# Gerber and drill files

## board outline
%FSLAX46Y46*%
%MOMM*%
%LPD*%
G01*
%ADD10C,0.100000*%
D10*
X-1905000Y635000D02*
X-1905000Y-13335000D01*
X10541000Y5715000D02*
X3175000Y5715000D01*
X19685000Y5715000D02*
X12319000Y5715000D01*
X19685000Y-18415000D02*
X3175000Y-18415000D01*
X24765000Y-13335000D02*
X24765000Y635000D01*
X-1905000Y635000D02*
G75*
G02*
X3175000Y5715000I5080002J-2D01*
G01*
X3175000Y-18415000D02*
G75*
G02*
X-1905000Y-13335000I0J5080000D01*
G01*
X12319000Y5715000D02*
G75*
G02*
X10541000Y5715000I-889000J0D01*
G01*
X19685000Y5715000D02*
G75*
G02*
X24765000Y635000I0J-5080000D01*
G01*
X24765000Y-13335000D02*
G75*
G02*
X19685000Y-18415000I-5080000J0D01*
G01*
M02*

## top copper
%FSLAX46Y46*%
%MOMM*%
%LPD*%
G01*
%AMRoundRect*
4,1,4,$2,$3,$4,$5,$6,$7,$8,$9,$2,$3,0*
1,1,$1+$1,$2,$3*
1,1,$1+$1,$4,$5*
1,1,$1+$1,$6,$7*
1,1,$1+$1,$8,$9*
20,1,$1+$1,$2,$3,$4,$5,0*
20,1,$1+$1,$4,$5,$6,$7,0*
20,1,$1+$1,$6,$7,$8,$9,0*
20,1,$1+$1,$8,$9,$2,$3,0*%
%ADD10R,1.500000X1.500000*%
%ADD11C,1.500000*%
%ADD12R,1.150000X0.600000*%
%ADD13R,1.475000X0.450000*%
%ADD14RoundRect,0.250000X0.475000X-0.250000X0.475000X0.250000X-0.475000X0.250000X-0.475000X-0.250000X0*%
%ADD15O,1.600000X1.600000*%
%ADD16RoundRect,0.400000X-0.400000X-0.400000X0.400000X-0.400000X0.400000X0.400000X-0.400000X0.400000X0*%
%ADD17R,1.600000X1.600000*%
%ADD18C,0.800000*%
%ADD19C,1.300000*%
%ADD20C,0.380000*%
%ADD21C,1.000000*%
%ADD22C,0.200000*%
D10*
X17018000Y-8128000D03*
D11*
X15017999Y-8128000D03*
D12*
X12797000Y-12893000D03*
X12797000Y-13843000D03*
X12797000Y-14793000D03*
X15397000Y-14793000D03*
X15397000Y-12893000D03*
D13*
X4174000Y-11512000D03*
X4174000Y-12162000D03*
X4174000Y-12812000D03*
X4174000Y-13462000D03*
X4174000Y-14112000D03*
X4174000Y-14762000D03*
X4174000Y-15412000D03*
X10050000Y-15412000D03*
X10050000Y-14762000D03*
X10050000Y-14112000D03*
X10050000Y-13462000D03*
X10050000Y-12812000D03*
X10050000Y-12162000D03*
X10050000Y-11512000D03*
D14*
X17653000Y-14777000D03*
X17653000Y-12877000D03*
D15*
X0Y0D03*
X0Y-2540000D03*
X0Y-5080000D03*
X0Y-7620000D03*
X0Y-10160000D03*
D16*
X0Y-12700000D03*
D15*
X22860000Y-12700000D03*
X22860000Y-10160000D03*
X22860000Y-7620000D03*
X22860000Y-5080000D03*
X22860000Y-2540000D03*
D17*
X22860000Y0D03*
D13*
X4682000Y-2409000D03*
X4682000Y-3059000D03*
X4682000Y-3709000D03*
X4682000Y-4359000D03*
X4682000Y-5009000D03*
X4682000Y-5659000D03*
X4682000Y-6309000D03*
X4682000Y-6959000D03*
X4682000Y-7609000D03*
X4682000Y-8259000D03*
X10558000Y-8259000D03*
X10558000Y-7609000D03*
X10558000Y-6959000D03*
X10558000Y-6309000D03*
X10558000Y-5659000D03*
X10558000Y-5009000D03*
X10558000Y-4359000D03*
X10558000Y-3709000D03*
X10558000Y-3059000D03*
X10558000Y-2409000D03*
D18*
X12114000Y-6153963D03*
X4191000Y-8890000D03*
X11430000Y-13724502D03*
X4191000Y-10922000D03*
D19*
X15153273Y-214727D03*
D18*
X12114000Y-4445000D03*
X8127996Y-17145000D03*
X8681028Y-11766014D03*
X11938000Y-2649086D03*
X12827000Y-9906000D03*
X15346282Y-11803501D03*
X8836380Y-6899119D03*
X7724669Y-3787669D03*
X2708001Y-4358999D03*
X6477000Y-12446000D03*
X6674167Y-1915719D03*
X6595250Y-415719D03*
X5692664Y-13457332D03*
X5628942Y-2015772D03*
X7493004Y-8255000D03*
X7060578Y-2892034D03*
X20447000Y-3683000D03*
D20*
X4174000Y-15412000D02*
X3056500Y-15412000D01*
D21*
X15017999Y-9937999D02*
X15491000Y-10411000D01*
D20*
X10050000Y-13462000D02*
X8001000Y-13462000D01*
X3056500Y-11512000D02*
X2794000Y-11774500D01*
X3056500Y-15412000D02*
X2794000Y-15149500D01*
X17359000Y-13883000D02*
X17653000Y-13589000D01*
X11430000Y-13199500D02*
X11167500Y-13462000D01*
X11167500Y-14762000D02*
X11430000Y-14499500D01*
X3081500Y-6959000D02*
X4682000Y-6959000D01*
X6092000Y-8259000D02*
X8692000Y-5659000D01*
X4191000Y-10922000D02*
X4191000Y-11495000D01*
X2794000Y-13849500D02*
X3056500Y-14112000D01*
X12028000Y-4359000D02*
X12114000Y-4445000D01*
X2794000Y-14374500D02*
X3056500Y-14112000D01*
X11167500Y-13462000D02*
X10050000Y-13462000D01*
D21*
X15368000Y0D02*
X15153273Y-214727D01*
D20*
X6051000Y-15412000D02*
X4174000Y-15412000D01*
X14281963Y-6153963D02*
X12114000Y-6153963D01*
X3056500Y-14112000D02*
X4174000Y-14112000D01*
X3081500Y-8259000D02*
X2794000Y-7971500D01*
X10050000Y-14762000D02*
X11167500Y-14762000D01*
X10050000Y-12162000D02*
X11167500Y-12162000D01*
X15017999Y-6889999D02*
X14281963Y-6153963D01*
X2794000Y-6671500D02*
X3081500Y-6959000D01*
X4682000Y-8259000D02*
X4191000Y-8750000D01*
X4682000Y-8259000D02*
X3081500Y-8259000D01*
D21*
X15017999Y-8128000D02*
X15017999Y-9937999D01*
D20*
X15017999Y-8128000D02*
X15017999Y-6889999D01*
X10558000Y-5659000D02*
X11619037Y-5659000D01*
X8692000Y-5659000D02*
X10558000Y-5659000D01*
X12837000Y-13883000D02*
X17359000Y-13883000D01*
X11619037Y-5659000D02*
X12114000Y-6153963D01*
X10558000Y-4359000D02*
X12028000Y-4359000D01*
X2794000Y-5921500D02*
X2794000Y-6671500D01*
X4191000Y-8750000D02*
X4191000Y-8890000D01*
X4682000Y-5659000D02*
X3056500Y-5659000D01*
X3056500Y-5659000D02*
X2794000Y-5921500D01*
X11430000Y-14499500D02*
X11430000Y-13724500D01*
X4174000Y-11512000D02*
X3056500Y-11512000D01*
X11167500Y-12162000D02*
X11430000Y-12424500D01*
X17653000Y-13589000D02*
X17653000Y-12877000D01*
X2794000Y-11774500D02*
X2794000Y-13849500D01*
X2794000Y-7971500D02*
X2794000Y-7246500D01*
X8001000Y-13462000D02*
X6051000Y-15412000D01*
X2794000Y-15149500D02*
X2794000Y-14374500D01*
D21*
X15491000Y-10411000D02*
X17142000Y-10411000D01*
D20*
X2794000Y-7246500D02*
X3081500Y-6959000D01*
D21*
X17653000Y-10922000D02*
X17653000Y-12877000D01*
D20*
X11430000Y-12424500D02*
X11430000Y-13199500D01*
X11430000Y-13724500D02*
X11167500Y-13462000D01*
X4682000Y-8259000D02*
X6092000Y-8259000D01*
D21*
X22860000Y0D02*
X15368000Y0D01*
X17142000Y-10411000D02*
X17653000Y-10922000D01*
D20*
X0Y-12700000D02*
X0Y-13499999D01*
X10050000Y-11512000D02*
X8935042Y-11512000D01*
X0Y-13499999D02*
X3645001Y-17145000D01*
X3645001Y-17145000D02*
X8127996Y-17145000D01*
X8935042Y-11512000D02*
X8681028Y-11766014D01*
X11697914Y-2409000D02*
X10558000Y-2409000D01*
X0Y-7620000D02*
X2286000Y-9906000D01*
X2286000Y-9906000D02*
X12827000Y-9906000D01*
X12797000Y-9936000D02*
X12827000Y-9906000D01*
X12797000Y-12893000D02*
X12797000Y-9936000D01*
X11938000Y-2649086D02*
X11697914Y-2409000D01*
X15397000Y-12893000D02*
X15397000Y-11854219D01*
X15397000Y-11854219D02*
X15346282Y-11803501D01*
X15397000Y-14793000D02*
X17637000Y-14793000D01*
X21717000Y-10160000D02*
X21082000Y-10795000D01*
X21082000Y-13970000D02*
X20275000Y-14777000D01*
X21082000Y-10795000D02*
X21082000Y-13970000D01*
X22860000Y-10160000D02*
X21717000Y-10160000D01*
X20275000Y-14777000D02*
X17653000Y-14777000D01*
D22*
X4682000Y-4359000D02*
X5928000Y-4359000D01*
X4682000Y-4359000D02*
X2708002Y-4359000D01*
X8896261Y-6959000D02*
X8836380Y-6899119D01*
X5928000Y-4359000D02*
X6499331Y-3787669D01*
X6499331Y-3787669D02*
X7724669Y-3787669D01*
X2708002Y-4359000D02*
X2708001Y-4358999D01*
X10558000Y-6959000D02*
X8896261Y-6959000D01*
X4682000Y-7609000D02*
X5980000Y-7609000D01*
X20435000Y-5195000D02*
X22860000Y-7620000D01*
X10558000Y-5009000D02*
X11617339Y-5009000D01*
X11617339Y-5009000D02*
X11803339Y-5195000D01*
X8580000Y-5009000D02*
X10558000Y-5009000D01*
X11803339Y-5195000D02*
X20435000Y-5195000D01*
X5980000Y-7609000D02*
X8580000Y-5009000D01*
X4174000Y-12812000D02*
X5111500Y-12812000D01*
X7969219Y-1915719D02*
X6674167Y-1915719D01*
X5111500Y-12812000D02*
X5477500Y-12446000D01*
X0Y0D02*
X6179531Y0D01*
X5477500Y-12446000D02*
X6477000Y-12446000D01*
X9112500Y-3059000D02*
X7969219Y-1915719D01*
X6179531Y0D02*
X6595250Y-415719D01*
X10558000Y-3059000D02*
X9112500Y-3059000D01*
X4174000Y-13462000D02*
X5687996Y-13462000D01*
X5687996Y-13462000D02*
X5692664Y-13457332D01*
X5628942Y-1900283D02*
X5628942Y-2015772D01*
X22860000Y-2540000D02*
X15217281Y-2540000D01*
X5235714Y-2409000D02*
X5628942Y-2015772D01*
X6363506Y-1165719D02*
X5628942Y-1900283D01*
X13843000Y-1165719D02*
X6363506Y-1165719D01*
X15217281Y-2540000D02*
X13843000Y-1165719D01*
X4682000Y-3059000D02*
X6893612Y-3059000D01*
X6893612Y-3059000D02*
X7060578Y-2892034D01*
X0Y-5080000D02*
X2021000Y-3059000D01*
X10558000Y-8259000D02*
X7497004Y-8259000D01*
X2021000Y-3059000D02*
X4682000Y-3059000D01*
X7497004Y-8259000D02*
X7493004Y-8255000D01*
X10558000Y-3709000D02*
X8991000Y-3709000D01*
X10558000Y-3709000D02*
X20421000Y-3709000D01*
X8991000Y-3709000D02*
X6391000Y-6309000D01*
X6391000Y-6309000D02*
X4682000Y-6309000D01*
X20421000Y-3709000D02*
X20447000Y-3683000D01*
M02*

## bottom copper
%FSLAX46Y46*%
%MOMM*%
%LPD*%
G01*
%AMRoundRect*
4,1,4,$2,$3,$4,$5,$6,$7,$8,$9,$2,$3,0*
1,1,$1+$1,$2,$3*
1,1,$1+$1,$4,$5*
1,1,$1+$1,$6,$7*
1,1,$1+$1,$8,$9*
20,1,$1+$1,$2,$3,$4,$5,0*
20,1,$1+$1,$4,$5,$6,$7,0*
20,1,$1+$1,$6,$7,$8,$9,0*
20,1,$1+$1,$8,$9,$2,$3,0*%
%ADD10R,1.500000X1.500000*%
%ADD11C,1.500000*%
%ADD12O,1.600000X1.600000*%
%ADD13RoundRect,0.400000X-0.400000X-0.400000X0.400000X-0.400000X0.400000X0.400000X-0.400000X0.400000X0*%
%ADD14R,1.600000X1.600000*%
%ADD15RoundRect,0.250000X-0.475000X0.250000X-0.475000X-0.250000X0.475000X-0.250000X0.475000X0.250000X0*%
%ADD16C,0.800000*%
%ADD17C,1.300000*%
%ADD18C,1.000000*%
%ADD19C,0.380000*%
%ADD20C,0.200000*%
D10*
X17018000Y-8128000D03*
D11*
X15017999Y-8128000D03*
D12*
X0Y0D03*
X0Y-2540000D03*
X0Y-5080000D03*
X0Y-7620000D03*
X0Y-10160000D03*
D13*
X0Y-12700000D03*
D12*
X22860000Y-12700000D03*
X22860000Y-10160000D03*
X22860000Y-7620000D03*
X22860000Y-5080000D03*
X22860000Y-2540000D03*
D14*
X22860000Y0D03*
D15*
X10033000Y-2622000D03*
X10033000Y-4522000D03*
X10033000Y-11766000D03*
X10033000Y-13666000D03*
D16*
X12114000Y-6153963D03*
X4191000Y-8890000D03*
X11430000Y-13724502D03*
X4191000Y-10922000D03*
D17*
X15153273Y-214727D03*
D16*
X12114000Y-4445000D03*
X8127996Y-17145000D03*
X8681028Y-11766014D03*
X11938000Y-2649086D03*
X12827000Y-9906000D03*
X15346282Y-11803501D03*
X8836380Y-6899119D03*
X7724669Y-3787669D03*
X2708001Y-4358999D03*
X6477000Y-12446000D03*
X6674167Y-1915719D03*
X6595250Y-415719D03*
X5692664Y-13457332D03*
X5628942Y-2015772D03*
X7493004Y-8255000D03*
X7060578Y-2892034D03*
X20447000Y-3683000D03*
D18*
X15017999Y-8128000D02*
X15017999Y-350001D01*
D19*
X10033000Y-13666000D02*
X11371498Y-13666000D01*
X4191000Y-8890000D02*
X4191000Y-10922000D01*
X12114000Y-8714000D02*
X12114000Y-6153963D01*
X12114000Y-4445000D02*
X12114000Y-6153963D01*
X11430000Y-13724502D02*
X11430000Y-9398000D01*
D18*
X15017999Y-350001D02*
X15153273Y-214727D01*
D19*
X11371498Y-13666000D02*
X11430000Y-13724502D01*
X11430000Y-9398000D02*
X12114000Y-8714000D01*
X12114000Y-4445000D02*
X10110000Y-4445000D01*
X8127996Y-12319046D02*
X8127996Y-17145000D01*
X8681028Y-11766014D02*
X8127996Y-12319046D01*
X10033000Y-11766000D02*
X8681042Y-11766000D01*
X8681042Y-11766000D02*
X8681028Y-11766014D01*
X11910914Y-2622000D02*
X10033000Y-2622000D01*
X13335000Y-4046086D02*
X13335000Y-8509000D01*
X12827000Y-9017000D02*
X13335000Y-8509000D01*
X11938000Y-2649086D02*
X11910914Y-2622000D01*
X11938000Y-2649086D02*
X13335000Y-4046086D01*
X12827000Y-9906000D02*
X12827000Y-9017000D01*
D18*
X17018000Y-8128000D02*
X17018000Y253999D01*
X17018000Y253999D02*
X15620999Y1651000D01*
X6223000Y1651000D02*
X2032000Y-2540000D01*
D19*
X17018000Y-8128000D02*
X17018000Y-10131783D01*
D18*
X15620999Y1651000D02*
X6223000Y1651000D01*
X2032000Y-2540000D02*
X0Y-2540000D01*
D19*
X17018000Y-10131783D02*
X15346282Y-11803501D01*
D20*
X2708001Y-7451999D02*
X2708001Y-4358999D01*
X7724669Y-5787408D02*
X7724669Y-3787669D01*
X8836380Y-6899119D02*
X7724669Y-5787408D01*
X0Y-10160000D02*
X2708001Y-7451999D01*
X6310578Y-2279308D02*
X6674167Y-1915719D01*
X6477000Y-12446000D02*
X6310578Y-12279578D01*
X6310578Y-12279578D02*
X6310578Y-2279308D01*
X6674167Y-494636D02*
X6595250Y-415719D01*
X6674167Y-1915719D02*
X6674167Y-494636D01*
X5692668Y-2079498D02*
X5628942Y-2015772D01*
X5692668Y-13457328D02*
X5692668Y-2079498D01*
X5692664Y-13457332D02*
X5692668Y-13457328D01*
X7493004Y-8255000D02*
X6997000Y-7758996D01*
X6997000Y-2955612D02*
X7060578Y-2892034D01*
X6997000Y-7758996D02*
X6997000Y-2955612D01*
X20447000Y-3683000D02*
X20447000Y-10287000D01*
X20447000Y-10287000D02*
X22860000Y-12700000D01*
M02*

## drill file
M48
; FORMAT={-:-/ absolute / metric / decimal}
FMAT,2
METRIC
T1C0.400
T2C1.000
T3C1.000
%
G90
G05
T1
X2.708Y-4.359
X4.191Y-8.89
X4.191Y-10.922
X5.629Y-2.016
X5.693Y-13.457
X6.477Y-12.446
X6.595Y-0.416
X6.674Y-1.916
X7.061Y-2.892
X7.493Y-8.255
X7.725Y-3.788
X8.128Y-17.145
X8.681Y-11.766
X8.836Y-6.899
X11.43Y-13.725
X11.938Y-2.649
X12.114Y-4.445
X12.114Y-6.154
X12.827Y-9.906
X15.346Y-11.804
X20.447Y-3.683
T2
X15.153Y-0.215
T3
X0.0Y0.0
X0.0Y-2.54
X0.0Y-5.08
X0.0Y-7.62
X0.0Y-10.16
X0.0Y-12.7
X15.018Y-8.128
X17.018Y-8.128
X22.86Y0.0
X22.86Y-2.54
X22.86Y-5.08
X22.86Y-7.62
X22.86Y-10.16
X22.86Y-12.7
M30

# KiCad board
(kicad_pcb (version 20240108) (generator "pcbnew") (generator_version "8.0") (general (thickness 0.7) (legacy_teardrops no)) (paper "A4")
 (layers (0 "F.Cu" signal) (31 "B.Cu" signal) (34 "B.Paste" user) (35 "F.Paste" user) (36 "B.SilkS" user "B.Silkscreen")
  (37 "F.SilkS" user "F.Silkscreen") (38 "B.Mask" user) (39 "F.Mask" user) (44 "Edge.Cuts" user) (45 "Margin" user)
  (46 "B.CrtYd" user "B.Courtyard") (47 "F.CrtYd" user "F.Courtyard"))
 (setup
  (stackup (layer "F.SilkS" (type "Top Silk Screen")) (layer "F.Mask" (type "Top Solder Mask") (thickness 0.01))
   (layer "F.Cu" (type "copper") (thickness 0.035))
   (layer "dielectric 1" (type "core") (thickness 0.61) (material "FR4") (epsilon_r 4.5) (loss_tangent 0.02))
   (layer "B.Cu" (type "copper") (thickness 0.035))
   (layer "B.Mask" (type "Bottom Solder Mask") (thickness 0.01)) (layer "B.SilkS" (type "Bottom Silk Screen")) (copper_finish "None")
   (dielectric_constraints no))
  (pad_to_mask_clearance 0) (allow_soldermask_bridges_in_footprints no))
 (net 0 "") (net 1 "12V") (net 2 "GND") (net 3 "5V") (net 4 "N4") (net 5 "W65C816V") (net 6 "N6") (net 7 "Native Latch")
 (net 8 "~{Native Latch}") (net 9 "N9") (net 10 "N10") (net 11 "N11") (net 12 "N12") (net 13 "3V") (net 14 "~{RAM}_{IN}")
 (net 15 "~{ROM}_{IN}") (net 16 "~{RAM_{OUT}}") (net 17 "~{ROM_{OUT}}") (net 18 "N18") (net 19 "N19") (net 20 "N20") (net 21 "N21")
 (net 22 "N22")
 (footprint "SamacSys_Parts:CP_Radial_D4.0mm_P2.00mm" (layer "F.Cu") (at 17.018 8.128 180)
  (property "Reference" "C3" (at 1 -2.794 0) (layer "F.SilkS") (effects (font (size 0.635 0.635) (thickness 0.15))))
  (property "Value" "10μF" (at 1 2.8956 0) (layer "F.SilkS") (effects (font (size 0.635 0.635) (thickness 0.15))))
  (pad "1" thru_hole rect (at 0 0 180) (size 1.5 1.5) (drill 1) (layers "*.Cu" "*.Mask") (remove_unused_layers no) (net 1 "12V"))
  (pad "2" thru_hole circle (at 2.000001 0 180) (size 1.5 1.5) (drill 1) (layers "*.Cu" "*.Mask") (remove_unused_layers no) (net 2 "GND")))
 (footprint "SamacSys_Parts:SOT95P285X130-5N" (layer "F.Cu") (at 14.097 13.843)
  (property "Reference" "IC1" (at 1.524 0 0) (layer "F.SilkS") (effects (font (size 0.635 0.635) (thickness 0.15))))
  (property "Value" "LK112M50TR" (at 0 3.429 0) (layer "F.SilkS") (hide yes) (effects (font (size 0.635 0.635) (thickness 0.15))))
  (pad "1" smd rect (at -1.3 -0.95 90) (size 0.6 1.15) (layers "F.Cu" "F.Paste" "F.Mask") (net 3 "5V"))
  (pad "2" smd rect (at -1.3 0 90) (size 0.6 1.15) (layers "F.Cu" "F.Paste" "F.Mask") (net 2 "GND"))
  (pad "3" smd rect (at -1.3 0.95 90) (size 0.6 1.15) (layers "F.Cu" "F.Paste" "F.Mask") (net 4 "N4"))
  (pad "4" smd rect (at 1.3 0.95 90) (size 0.6 1.15) (layers "F.Cu" "F.Paste" "F.Mask") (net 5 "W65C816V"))
  (pad "5" smd rect (at 1.3 -0.95 90) (size 0.6 1.15) (layers "F.Cu" "F.Paste" "F.Mask") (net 1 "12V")))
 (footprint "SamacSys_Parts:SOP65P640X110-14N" (layer "F.Cu") (at 7.112 13.462)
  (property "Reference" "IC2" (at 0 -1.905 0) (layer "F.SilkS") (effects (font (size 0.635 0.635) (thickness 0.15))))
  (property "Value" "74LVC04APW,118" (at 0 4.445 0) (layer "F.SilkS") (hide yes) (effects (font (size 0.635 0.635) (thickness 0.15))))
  (pad "1" smd rect (at -2.938 -1.95 90) (size 0.45 1.475) (layers "F.Cu" "F.Paste" "F.Mask") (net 2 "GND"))
  (pad "2" smd rect (at -2.938 -1.3 90) (size 0.45 1.475) (layers "F.Cu" "F.Paste" "F.Mask") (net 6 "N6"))
  (pad "3" smd rect (at -2.938 -0.65 90) (size 0.45 1.475) (layers "F.Cu" "F.Paste" "F.Mask") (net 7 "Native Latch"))
  (pad "4" smd rect (at -2.938 0 90) (size 0.45 1.475) (layers "F.Cu" "F.Paste" "F.Mask") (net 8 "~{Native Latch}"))
  (pad "5" smd rect (at -2.938 0.65 90) (size 0.45 1.475) (layers "F.Cu" "F.Paste" "F.Mask") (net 2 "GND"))
  (pad "6" smd rect (at -2.938 1.3 90) (size 0.45 1.475) (layers "F.Cu" "F.Paste" "F.Mask") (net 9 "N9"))
  (pad "7" smd rect (at -2.938 1.95 90) (size 0.45 1.475) (layers "F.Cu" "F.Paste" "F.Mask") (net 2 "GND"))
  (pad "8" smd rect (at 2.938 1.95 90) (size 0.45 1.475) (layers "F.Cu" "F.Paste" "F.Mask") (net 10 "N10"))
  (pad "9" smd rect (at 2.938 1.3 90) (size 0.45 1.475) (layers "F.Cu" "F.Paste" "F.Mask") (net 2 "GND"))
  (pad "10" smd rect (at 2.938 0.65 90) (size 0.45 1.475) (layers "F.Cu" "F.Paste" "F.Mask") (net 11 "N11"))
  (pad "11" smd rect (at 2.938 0 90) (size 0.45 1.475) (layers "F.Cu" "F.Paste" "F.Mask") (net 2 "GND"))
  (pad "12" smd rect (at 2.938 -0.65 90) (size 0.45 1.475) (layers "F.Cu" "F.Paste" "F.Mask") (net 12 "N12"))
  (pad "13" smd rect (at 2.938 -1.3 90) (size 0.45 1.475) (layers "F.Cu" "F.Paste" "F.Mask") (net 2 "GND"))
  (pad "14" smd rect (at 2.938 -1.95 90) (size 0.45 1.475) (layers "F.Cu" "F.Paste" "F.Mask") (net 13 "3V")))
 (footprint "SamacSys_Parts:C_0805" (layer "F.Cu") (at 17.653 13.843)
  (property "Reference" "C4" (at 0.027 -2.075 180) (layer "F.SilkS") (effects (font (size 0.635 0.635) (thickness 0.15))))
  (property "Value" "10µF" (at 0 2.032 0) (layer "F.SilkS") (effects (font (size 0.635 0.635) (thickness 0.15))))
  (pad "1" smd roundrect (at 0 0.934 90) (size 1 1.45) (layers "F.Cu" "F.Paste" "F.Mask") (roundrect_rratio 0.25) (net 5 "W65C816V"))
  (pad "2" smd roundrect (at 0 -0.966 90) (size 1 1.45) (layers "F.Cu" "F.Paste" "F.Mask") (roundrect_rratio 0.25) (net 2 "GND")))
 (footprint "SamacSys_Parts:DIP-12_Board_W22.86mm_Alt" (layer "F.Cu") (at 0 0)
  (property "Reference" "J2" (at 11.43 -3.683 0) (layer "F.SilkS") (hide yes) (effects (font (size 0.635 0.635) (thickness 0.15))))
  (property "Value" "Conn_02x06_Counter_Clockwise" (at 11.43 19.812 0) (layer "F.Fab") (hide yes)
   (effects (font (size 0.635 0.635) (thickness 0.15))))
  (fp_line (start -1.905 -0.635) (end -1.905 13.335) (stroke (width 0.1) (type solid)) (layer "Edge.Cuts"))
  (fp_line (start 10.541 -5.715) (end 3.175 -5.715) (stroke (width 0.1) (type solid)) (layer "Edge.Cuts"))
  (fp_line (start 19.685 -5.715) (end 12.319 -5.715) (stroke (width 0.1) (type solid)) (layer "Edge.Cuts"))
  (fp_line (start 19.685 18.415) (end 3.175 18.415) (stroke (width 0.1) (type solid)) (layer "Edge.Cuts"))
  (fp_line (start 24.765 13.335) (end 24.765 -0.635) (stroke (width 0.1) (type solid)) (layer "Edge.Cuts"))
  (fp_arc (start -1.905 -0.635) (mid -0.417102 -4.227102) (end 3.175 -5.715) (stroke (width 0.1) (type solid)) (layer "Edge.Cuts"))
  (fp_arc (start 3.175 18.415) (mid -0.417102 16.927102) (end -1.905 13.335) (stroke (width 0.1) (type solid)) (layer "Edge.Cuts"))
  (fp_arc (start 12.319 -5.715) (mid 11.43 -4.826) (end 10.541 -5.715) (stroke (width 0.1) (type default)) (layer "Edge.Cuts"))
  (fp_arc (start 19.685 -5.715) (mid 23.277102 -4.227102) (end 24.765 -0.635) (stroke (width 0.1) (type solid)) (layer "Edge.Cuts"))
  (fp_arc (start 24.765 13.335) (mid 23.277102 16.927102) (end 19.685 18.415) (stroke (width 0.1) (type solid)) (layer "Edge.Cuts"))
  (pad "1" thru_hole oval (at 0 0) (size 1.6 1.6) (drill 1) (layers "*.Cu" "*.Mask") (remove_unused_layers no) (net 7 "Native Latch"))
  (pad "2" thru_hole oval (at 0 2.54) (size 1.6 1.6) (drill 1) (layers "*.Cu" "*.Mask") (remove_unused_layers no) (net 1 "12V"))
  (pad "3" thru_hole oval (at 0 5.08) (size 1.6 1.6) (drill 1) (layers "*.Cu" "*.Mask") (remove_unused_layers no) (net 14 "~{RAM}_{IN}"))
  (pad "4" thru_hole oval (at 0 7.62) (size 1.6 1.6) (drill 1) (layers "*.Cu" "*.Mask") (remove_unused_layers no) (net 3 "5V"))
  (pad "5" thru_hole oval (at 0 10.16) (size 1.6 1.6) (drill 1) (layers "*.Cu" "*.Mask") (remove_unused_layers no) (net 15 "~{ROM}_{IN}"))
  (pad "6" thru_hole roundrect (at 0 12.7) (size 1.6 1.6) (drill 1) (layers "*.Cu" "*.Mask") (remove_unused_layers no)
   (roundrect_rratio 0.25) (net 13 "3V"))
  (pad "7" thru_hole oval (at 22.86 12.7 180) (size 1.6 1.6) (drill 1) (layers "*.Cu" "*.Mask") (remove_unused_layers no)
   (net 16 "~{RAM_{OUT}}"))
  (pad "8" thru_hole oval (at 22.86 10.16 180) (size 1.6 1.6) (drill 1) (layers "*.Cu" "*.Mask") (remove_unused_layers no)
   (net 5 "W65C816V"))
  (pad "9" thru_hole oval (at 22.86 7.62) (size 1.6 1.6) (drill 1) (layers "*.Cu" "*.Mask") (remove_unused_layers no)
   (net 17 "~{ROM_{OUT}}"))
  (pad "10" thru_hole oval (at 22.86 5.08) (size 1.6 1.6) (drill 1) (layers "*.Cu" "*.Mask") (remove_unused_layers no) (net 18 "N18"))
  (pad "11" thru_hole oval (at 22.86 2.54) (size 1.6 1.6) (drill 1) (layers "*.Cu" "*.Mask") (remove_unused_layers no)
   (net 8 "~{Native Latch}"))
  (pad "12" thru_hole rect (at 22.86 0) (size 1.6 1.6) (drill 1) (layers "*.Cu" "*.Mask") (remove_unused_layers no) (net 2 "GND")))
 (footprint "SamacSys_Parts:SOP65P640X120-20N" (layer "F.Cu") (at 7.62 5.334)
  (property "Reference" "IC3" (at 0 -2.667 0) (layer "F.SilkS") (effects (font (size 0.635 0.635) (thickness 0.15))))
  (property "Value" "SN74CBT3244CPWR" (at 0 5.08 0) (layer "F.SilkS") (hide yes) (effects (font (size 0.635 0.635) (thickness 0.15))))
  (pad "1" smd rect (at -2.938 -2.925 90) (size 0.45 1.475) (layers "F.Cu" "F.Paste" "F.Mask") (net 8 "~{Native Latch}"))
  (pad "2" smd rect (at -2.938 -2.275 90) (size 0.45 1.475) (layers "F.Cu" "F.Paste" "F.Mask") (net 14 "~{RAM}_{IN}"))
  (pad "3" smd rect (at -2.938 -1.625 90) (size 0.45 1.475) (layers "F.Cu" "F.Paste" "F.Mask") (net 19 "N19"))
  (pad "4" smd rect (at -2.938 -0.975 90) (size 0.45 1.475) (layers "F.Cu" "F.Paste" "F.Mask") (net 15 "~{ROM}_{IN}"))
  (pad "5" smd rect (at -2.938 -0.325 90) (size 0.45 1.475) (layers "F.Cu" "F.Paste" "F.Mask") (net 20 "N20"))
  (pad "6" smd rect (at -2.938 0.325 90) (size 0.45 1.475) (layers "F.Cu" "F.Paste" "F.Mask") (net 2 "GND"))
  (pad "7" smd rect (at -2.938 0.975 90) (size 0.45 1.475) (layers "F.Cu" "F.Paste" "F.Mask") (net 16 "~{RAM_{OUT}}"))
  (pad "8" smd rect (at -2.938 1.625 90) (size 0.45 1.475) (layers "F.Cu" "F.Paste" "F.Mask") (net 2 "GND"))
  (pad "9" smd rect (at -2.938 2.275 90) (size 0.45 1.475) (layers "F.Cu" "F.Paste" "F.Mask") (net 17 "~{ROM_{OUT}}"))
  (pad "10" smd rect (at -2.938 2.925 90) (size 0.45 1.475) (layers "F.Cu" "F.Paste" "F.Mask") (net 2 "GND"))
  (pad "11" smd rect (at 2.938 2.925 90) (size 0.45 1.475) (layers "F.Cu" "F.Paste" "F.Mask") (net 14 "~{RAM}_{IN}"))
  (pad "12" smd rect (at 2.938 2.275 90) (size 0.45 1.475) (layers "F.Cu" "F.Paste" "F.Mask") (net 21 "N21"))
  (pad "13" smd rect (at 2.938 1.625 90) (size 0.45 1.475) (layers "F.Cu" "F.Paste" "F.Mask") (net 15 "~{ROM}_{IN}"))
  (pad "14" smd rect (at 2.938 0.975 90) (size 0.45 1.475) (layers "F.Cu" "F.Paste" "F.Mask") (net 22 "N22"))
  (pad "15" smd rect (at 2.938 0.325 90) (size 0.45 1.475) (layers "F.Cu" "F.Paste" "F.Mask") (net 2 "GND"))
  (pad "16" smd rect (at 2.938 -0.325 90) (size 0.45 1.475) (layers "F.Cu" "F.Paste" "F.Mask") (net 17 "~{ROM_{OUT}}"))
  (pad "17" smd rect (at 2.938 -0.975 90) (size 0.45 1.475) (layers "F.Cu" "F.Paste" "F.Mask") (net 2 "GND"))
  (pad "18" smd rect (at 2.938 -1.625 90) (size 0.45 1.475) (layers "F.Cu" "F.Paste" "F.Mask") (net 16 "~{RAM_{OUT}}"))
  (pad "19" smd rect (at 2.938 -2.275 90) (size 0.45 1.475) (layers "F.Cu" "F.Paste" "F.Mask") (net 7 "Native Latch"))
  (pad "20" smd rect (at 2.938 -2.925 90) (size 0.45 1.475) (layers "F.Cu" "F.Paste" "F.Mask") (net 3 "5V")))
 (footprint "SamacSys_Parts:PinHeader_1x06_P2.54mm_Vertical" (layer "B.Cu") (at 22.86 0 180)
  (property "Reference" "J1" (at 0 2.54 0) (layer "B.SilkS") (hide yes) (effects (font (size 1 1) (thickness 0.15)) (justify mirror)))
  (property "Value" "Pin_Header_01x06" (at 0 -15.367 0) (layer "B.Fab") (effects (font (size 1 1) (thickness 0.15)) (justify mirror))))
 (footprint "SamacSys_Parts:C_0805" (layer "B.Cu") (at 10.033 3.556)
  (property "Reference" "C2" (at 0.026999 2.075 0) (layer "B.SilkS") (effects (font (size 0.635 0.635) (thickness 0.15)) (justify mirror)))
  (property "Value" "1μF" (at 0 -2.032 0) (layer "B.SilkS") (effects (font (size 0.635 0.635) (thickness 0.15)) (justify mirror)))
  (pad "1" smd roundrect (at 0 -0.934 270) (size 1 1.45) (layers "B.Cu" "B.Paste" "B.Mask") (roundrect_rratio 0.25) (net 3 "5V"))
  (pad "2" smd roundrect (at 0 0.966 270) (size 1 1.45) (layers "B.Cu" "B.Paste" "B.Mask") (roundrect_rratio 0.25) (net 2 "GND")))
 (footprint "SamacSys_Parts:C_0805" (layer "B.Cu") (at 10.033 12.7)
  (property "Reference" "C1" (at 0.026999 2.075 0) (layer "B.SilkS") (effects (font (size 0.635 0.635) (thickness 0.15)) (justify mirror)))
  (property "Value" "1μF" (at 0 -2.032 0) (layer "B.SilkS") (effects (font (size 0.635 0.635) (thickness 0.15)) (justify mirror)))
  (pad "1" smd roundrect (at 0 -0.934 270) (size 1 1.45) (layers "B.Cu" "B.Paste" "B.Mask") (roundrect_rratio 0.25) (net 13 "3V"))
  (pad "2" smd roundrect (at 0 0.966 270) (size 1 1.45) (layers "B.Cu" "B.Paste" "B.Mask") (roundrect_rratio 0.25) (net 2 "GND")))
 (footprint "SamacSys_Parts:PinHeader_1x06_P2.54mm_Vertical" (layer "B.Cu") (at 0 0 180)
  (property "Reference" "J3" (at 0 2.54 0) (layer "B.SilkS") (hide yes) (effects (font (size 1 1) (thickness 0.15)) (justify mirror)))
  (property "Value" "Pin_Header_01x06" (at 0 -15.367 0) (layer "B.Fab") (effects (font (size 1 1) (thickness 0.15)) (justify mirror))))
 (segment (start 4.174 15.412) (end 3.0565 15.412) (width 0.38) (layer "F.Cu") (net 2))
 (segment (start 15.017999 9.937999) (end 15.491 10.411) (width 1) (layer "F.Cu") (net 2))
 (segment (start 10.05 13.462) (end 8.001 13.462) (width 0.38) (layer "F.Cu") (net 2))
 (segment (start 3.0565 11.512) (end 2.794 11.7745) (width 0.38) (layer "F.Cu") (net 2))
 (segment (start 3.0565 15.412) (end 2.794 15.1495) (width 0.38) (layer "F.Cu") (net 2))
 (segment (start 17.359 13.883) (end 17.653 13.589) (width 0.38) (layer "F.Cu") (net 2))
 (segment (start 11.43 13.1995) (end 11.1675 13.462) (width 0.38) (layer "F.Cu") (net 2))
 (segment (start 11.1675 14.762) (end 11.43 14.4995) (width 0.38) (layer "F.Cu") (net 2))
 (segment (start 3.0815 6.959) (end 4.682 6.959) (width 0.38) (layer "F.Cu") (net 2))
 (segment (start 6.092 8.259) (end 8.692 5.659) (width 0.38) (layer "F.Cu") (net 2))
 (segment (start 4.191 10.922) (end 4.191 11.495) (width 0.38) (layer "F.Cu") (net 2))
 (segment (start 2.794 13.8495) (end 3.0565 14.112) (width 0.38) (layer "F.Cu") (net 2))
 (segment (start 12.028 4.359) (end 12.114 4.445) (width 0.38) (layer "F.Cu") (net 2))
 (segment (start 2.794 14.3745) (end 3.0565 14.112) (width 0.38) (layer "F.Cu") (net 2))
 (segment (start 11.1675 13.462) (end 10.05 13.462) (width 0.38) (layer "F.Cu") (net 2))
 (segment (start 15.368 0) (end 15.153273 0.214727) (width 1) (layer "F.Cu") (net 2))
 (segment (start 6.051 15.412) (end 4.174 15.412) (width 0.38) (layer "F.Cu") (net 2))
 (segment (start 14.281963 6.153963) (end 12.114 6.153963) (width 0.38) (layer "F.Cu") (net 2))
 (segment (start 3.0565 14.112) (end 4.174 14.112) (width 0.38) (layer "F.Cu") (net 2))
 (segment (start 3.0815 8.259) (end 2.794 7.9715) (width 0.38) (layer "F.Cu") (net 2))
 (segment (start 10.05 14.762) (end 11.1675 14.762) (width 0.38) (layer "F.Cu") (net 2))
 (segment (start 10.05 12.162) (end 11.1675 12.162) (width 0.38) (layer "F.Cu") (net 2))
 (segment (start 15.017999 6.889999) (end 14.281963 6.153963) (width 0.38) (layer "F.Cu") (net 2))
 (segment (start 2.794 6.6715) (end 3.0815 6.959) (width 0.38) (layer "F.Cu") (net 2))
 (segment (start 4.682 8.259) (end 4.191 8.75) (width 0.38) (layer "F.Cu") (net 2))
 (segment (start 4.682 8.259) (end 3.0815 8.259) (width 0.38) (layer "F.Cu") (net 2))
 (segment (start 15.017999 8.128) (end 15.017999 9.937999) (width 1) (layer "F.Cu") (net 2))
 (segment (start 15.017999 8.128) (end 15.017999 6.889999) (width 0.38) (layer "F.Cu") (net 2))
 (segment (start 10.558 5.659) (end 11.619037 5.659) (width 0.38) (layer "F.Cu") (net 2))
 (segment (start 8.692 5.659) (end 10.558 5.659) (width 0.38) (layer "F.Cu") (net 2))
 (segment (start 12.837 13.883) (end 17.359 13.883) (width 0.38) (layer "F.Cu") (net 2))
 (segment (start 11.619037 5.659) (end 12.114 6.153963) (width 0.38) (layer "F.Cu") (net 2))
 (segment (start 10.558 4.359) (end 12.028 4.359) (width 0.38) (layer "F.Cu") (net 2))
 (segment (start 2.794 5.9215) (end 2.794 6.6715) (width 0.38) (layer "F.Cu") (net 2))
 (segment (start 4.191 8.75) (end 4.191 8.89) (width 0.38) (layer "F.Cu") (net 2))
 (segment (start 4.682 5.659) (end 3.0565 5.659) (width 0.38) (layer "F.Cu") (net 2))
 (segment (start 3.0565 5.659) (end 2.794 5.9215) (width 0.38) (layer "F.Cu") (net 2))
 (segment (start 11.43 14.4995) (end 11.43 13.7245) (width 0.38) (layer "F.Cu") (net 2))
 (segment (start 4.174 11.512) (end 3.0565 11.512) (width 0.38) (layer "F.Cu") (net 2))
 (segment (start 11.1675 12.162) (end 11.43 12.4245) (width 0.38) (layer "F.Cu") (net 2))
 (segment (start 17.653 13.589) (end 17.653 12.877) (width 0.38) (layer "F.Cu") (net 2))
 (segment (start 2.794 11.7745) (end 2.794 13.8495) (width 0.38) (layer "F.Cu") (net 2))
 (segment (start 2.794 7.9715) (end 2.794 7.2465) (width 0.38) (layer "F.Cu") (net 2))
 (segment (start 8.001 13.462) (end 6.051 15.412) (width 0.38) (layer "F.Cu") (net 2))
 (segment (start 2.794 15.1495) (end 2.794 14.3745) (width 0.38) (layer "F.Cu") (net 2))
 (segment (start 15.491 10.411) (end 17.142 10.411) (width 1) (layer "F.Cu") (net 2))
 (segment (start 2.794 7.2465) (end 3.0815 6.959) (width 0.38) (layer "F.Cu") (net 2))
 (segment (start 17.653 10.922) (end 17.653 12.877) (width 1) (layer "F.Cu") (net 2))
 (segment (start 11.43 12.4245) (end 11.43 13.1995) (width 0.38) (layer "F.Cu") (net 2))
 (segment (start 11.43 13.7245) (end 11.1675 13.462) (width 0.38) (layer "F.Cu") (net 2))
 (segment (start 4.682 8.259) (end 6.092 8.259) (width 0.38) (layer "F.Cu") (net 2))
 (segment (start 22.86 0) (end 15.368 0) (width 1) (layer "F.Cu") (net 2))
 (segment (start 17.142 10.411) (end 17.653 10.922) (width 1) (layer "F.Cu") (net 2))
 (via (at 12.114 6.153963) (size 0.8) (drill 0.4) (layers "F.Cu" "B.Cu") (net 2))
 (via (at 4.191 8.89) (size 0.8) (drill 0.4) (layers "F.Cu" "B.Cu") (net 2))
 (via (at 11.43 13.724502) (size 0.8) (drill 0.4) (layers "F.Cu" "B.Cu") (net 2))
 (via (at 4.191 10.922) (size 0.8) (drill 0.4) (layers "F.Cu" "B.Cu") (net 2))
 (via (at 15.153273 0.214727) (size 1.3) (drill 1) (layers "F.Cu" "B.Cu") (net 2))
 (via (at 12.114 4.445) (size 0.8) (drill 0.4) (layers "F.Cu" "B.Cu") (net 2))
 (segment (start 15.017999 8.128) (end 15.017999 0.350001) (width 1) (layer "B.Cu") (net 2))
 (segment (start 10.033 13.666) (end 11.371498 13.666) (width 0.38) (layer "B.Cu") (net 2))
 (segment (start 4.191 8.89) (end 4.191 10.922) (width 0.38) (layer "B.Cu") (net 2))
 (segment (start 12.114 8.714) (end 12.114 6.153963) (width 0.38) (layer "B.Cu") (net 2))
 (segment (start 12.114 4.445) (end 12.114 6.153963) (width 0.38) (layer "B.Cu") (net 2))
 (segment (start 11.43 13.724502) (end 11.43 9.398) (width 0.38) (layer "B.Cu") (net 2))
 (segment (start 15.017999 0.350001) (end 15.153273 0.214727) (width 1) (layer "B.Cu") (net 2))
 (segment (start 11.371498 13.666) (end 11.43 13.724502) (width 0.38) (layer "B.Cu") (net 2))
 (segment (start 11.43 9.398) (end 12.114 8.714) (width 0.38) (layer "B.Cu") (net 2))
 (segment (start 12.114 4.445) (end 10.11 4.445) (width 0.38) (layer "B.Cu") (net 2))
 (segment (start 0 12.7) (end 0 13.499999) (width 0.38) (layer "F.Cu") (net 13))
 (segment (start 10.05 11.512) (end 8.935042 11.512) (width 0.38) (layer "F.Cu") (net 13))
 (segment (start 0 13.499999) (end 3.645001 17.145) (width 0.38) (layer "F.Cu") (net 13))
 (segment (start 3.645001 17.145) (end 8.127996 17.145) (width 0.38) (layer "F.Cu") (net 13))
 (segment (start 8.935042 11.512) (end 8.681028 11.766014) (width 0.38) (layer "F.Cu") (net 13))
 (via (at 8.127996 17.145) (size 0.8) (drill 0.4) (layers "F.Cu" "B.Cu") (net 13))
 (via (at 8.681028 11.766014) (size 0.8) (drill 0.4) (layers "F.Cu" "B.Cu") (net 13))
 (segment (start 8.127996 12.319046) (end 8.127996 17.145) (width 0.38) (layer "B.Cu") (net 13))
 (segment (start 8.681028 11.766014) (end 8.127996 12.319046) (width 0.38) (layer "B.Cu") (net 13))
 (segment (start 10.033 11.766) (end 8.681042 11.766) (width 0.38) (layer "B.Cu") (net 13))
 (segment (start 8.681042 11.766) (end 8.681028 11.766014) (width 0.38) (layer "B.Cu") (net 13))
 (segment (start 11.697914 2.409) (end 10.558 2.409) (width 0.38) (layer "F.Cu") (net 3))
 (segment (start 0 7.62) (end 2.286 9.906) (width 0.38) (layer "F.Cu") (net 3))
 (segment (start 2.286 9.906) (end 12.827 9.906) (width 0.38) (layer "F.Cu") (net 3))
 (segment (start 12.797 9.936) (end 12.827 9.906) (width 0.38) (layer "F.Cu") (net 3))
 (segment (start 12.797 12.893) (end 12.797 9.936) (width 0.38) (layer "F.Cu") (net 3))
 (segment (start 11.938 2.649086) (end 11.697914 2.409) (width 0.38) (layer "F.Cu") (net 3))
 (via (at 11.938 2.649086) (size 0.8) (drill 0.4) (layers "F.Cu" "B.Cu") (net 3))
 (via (at 12.827 9.906) (size 0.8) (drill 0.4) (layers "F.Cu" "B.Cu") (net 3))
 (segment (start 11.910914 2.622) (end 10.033 2.622) (width 0.38) (layer "B.Cu") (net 3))
 (segment (start 13.335 4.046086) (end 13.335 8.509) (width 0.38) (layer "B.Cu") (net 3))
 (segment (start 12.827 9.017) (end 13.335 8.509) (width 0.38) (layer "B.Cu") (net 3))
 (segment (start 11.938 2.649086) (end 11.910914 2.622) (width 0.38) (layer "B.Cu") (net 3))
 (segment (start 11.938 2.649086) (end 13.335 4.046086) (width 0.38) (layer "B.Cu") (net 3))
 (segment (start 12.827 9.906) (end 12.827 9.017) (width 0.38) (layer "B.Cu") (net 3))
 (segment (start 15.397 12.893) (end 15.397 11.854219) (width 0.38) (layer "F.Cu") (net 1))
 (segment (start 15.397 11.854219) (end 15.346282 11.803501) (width 0.38) (layer "F.Cu") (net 1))
 (via (at 15.346282 11.803501) (size 0.8) (drill 0.4) (layers "F.Cu" "B.Cu") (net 1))
 (segment (start 17.018 8.128) (end 17.018 -0.253999) (width 1) (layer "B.Cu") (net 1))
 (segment (start 17.018 -0.253999) (end 15.620999 -1.651) (width 1) (layer "B.Cu") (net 1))
 (segment (start 6.223 -1.651) (end 2.032 2.54) (width 1) (layer "B.Cu") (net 1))
 (segment (start 17.018 8.128) (end 17.018 10.131783) (width 0.38) (layer "B.Cu") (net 1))
 (segment (start 15.620999 -1.651) (end 6.223 -1.651) (width 1) (layer "B.Cu") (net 1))
 (segment (start 2.032 2.54) (end 0 2.54) (width 1) (layer "B.Cu") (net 1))
 (segment (start 17.018 10.131783) (end 15.346282 11.803501) (width 0.38) (layer "B.Cu") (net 1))
 (segment (start 15.397 14.793) (end 17.637 14.793) (width 0.38) (layer "F.Cu") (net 5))
 (segment (start 21.717 10.16) (end 21.082 10.795) (width 0.38) (layer "F.Cu") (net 5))
 (segment (start 21.082 13.97) (end 20.275 14.777) (width 0.38) (layer "F.Cu") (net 5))
 (segment (start 21.082 10.795) (end 21.082 13.97) (width 0.38) (layer "F.Cu") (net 5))
 (segment (start 22.86 10.16) (end 21.717 10.16) (width 0.38) (layer "F.Cu") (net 5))
 (segment (start 20.275 14.777) (end 17.653 14.777) (width 0.38) (layer "F.Cu") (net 5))
 (segment (start 4.682 4.359) (end 5.928 4.359) (width 0.2) (layer "F.Cu") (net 15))
 (segment (start 4.682 4.359) (end 2.708002 4.359) (width 0.2) (layer "F.Cu") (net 15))
 (segment (start 8.896261 6.959) (end 8.83638 6.899119) (width 0.2) (layer "F.Cu") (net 15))
 (segment (start 5.928 4.359) (end 6.499331 3.787669) (width 0.2) (layer "F.Cu") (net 15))
 (segment (start 6.499331 3.787669) (end 7.724669 3.787669) (width 0.2) (layer "F.Cu") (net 15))
 (segment (start 2.708002 4.359) (end 2.708001 4.358999) (width 0.2) (layer "F.Cu") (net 15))
 (segment (start 10.558 6.959) (end 8.896261 6.959) (width 0.2) (layer "F.Cu") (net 15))
 (via (at 8.83638 6.899119) (size 0.8) (drill 0.4) (layers "F.Cu" "B.Cu") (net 15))
 (via (at 7.724669 3.787669) (size 0.8) (drill 0.4) (layers "F.Cu" "B.Cu") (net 15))
 (via (at 2.708001 4.358999) (size 0.8) (drill 0.4) (layers "F.Cu" "B.Cu") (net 15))
 (segment (start 2.708001 7.451999) (end 2.708001 4.358999) (width 0.2) (layer "B.Cu") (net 15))
 (segment (start 7.724669 5.787408) (end 7.724669 3.787669) (width 0.2) (layer "B.Cu") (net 15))
 (segment (start 8.83638 6.899119) (end 7.724669 5.787408) (width 0.2) (layer "B.Cu") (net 15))
 (segment (start 0 10.16) (end 2.708001 7.451999) (width 0.2) (layer "B.Cu") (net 15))
 (segment (start 4.682 7.609) (end 5.98 7.609) (width 0.2) (layer "F.Cu") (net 17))
 (segment (start 20.435 5.195) (end 22.86 7.62) (width 0.2) (layer "F.Cu") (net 17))
 (segment (start 10.558 5.009) (end 11.617339 5.009) (width 0.2) (layer "F.Cu") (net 17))
 (segment (start 11.617339 5.009) (end 11.803339 5.195) (width 0.2) (layer "F.Cu") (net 17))
 (segment (start 8.58 5.009) (end 10.558 5.009) (width 0.2) (layer "F.Cu") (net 17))
 (segment (start 11.803339 5.195) (end 20.435 5.195) (width 0.2) (layer "F.Cu") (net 17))
 (segment (start 5.98 7.609) (end 8.58 5.009) (width 0.2) (layer "F.Cu") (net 17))
 (segment (start 4.174 12.812) (end 5.1115 12.812) (width 0.2) (layer "F.Cu") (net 7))
 (segment (start 7.969219 1.915719) (end 6.674167 1.915719) (width 0.2) (layer "F.Cu") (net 7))
 (segment (start 5.1115 12.812) (end 5.4775 12.446) (width 0.2) (layer "F.Cu") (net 7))
 (segment (start 0 0) (end 6.179531 0) (width 0.2) (layer "F.Cu") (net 7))
 (segment (start 5.4775 12.446) (end 6.477 12.446) (width 0.2) (layer "F.Cu") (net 7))
 (segment (start 9.1125 3.059) (end 7.969219 1.915719) (width 0.2) (layer "F.Cu") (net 7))
 (segment (start 6.179531 0) (end 6.59525 0.415719) (width 0.2) (layer "F.Cu") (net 7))
 (segment (start 10.558 3.059) (end 9.1125 3.059) (width 0.2) (layer "F.Cu") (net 7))
 (via (at 6.477 12.446) (size 0.8) (drill 0.4) (layers "F.Cu" "B.Cu") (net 7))
 (via (at 6.674167 1.915719) (size 0.8) (drill 0.4) (layers "F.Cu" "B.Cu") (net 7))
 (via (at 6.59525 0.415719) (size 0.8) (drill 0.4) (layers "F.Cu" "B.Cu") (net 7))
 (segment (start 6.310578 2.279308) (end 6.674167 1.915719) (width 0.2) (layer "B.Cu") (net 7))
 (segment (start 6.477 12.446) (end 6.310578 12.279578) (width 0.2) (layer "B.Cu") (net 7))
 (segment (start 6.310578 12.279578) (end 6.310578 2.279308) (width 0.2) (layer "B.Cu") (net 7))
 (segment (start 6.674167 0.494636) (end 6.59525 0.415719) (width 0.2) (layer "B.Cu") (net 7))
 (segment (start 6.674167 1.915719) (end 6.674167 0.494636) (width 0.2) (layer "B.Cu") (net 7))
 (segment (start 4.174 13.462) (end 5.687996 13.462) (width 0.2) (layer "F.Cu") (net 8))
 (segment (start 5.687996 13.462) (end 5.692664 13.457332) (width 0.2) (layer "F.Cu") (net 8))
 (segment (start 5.628942 1.900283) (end 5.628942 2.015772) (width 0.2) (layer "F.Cu") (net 8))
 (segment (start 22.86 2.54) (end 15.217281 2.54) (width 0.2) (layer "F.Cu") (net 8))
 (segment (start 5.235714 2.409) (end 5.628942 2.015772) (width 0.2) (layer "F.Cu") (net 8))
 (segment (start 6.363506 1.165719) (end 5.628942 1.900283) (width 0.2) (layer "F.Cu") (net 8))
 (segment (start 13.843 1.165719) (end 6.363506 1.165719) (width 0.2) (layer "F.Cu") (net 8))
 (segment (start 15.217281 2.54) (end 13.843 1.165719) (width 0.2) (layer "F.Cu") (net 8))
 (via (at 5.692664 13.457332) (size 0.8) (drill 0.4) (layers "F.Cu" "B.Cu") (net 8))
 (via (at 5.628942 2.015772) (size 0.8) (drill 0.4) (layers "F.Cu" "B.Cu") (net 8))
 (segment (start 5.692668 2.079498) (end 5.628942 2.015772) (width 0.2) (layer "B.Cu") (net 8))
 (segment (start 5.692668 13.457328) (end 5.692668 2.079498) (width 0.2) (layer "B.Cu") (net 8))
 (segment (start 5.692664 13.457332) (end 5.692668 13.457328) (width 0.2) (layer "B.Cu") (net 8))
 (segment (start 4.682 3.059) (end 6.893612 3.059) (width 0.2) (layer "F.Cu") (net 14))
 (segment (start 6.893612 3.059) (end 7.060578 2.892034) (width 0.2) (layer "F.Cu") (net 14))
 (segment (start 0 5.08) (end 2.021 3.059) (width 0.2) (layer "F.Cu") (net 14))
 (segment (start 10.558 8.259) (end 7.497004 8.259) (width 0.2) (layer "F.Cu") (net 14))
 (segment (start 2.021 3.059) (end 4.682 3.059) (width 0.2) (layer "F.Cu") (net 14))
 (segment (start 7.497004 8.259) (end 7.493004 8.255) (width 0.2) (layer "F.Cu") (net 14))
 (via (at 7.493004 8.255) (size 0.8) (drill 0.4) (layers "F.Cu" "B.Cu") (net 14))
 (via (at 7.060578 2.892034) (size 0.8) (drill 0.4) (layers "F.Cu" "B.Cu") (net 14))
 (segment (start 7.493004 8.255) (end 6.997 7.758996) (width 0.2) (layer "B.Cu") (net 14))
 (segment (start 6.997 2.955612) (end 7.060578 2.892034) (width 0.2) (layer "B.Cu") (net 14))
 (segment (start 6.997 7.758996) (end 6.997 2.955612) (width 0.2) (layer "B.Cu") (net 14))
 (segment (start 10.558 3.709) (end 8.991 3.709) (width 0.2) (layer "F.Cu") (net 16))
 (segment (start 10.558 3.709) (end 20.421 3.709) (width 0.2) (layer "F.Cu") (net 16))
 (segment (start 8.991 3.709) (end 6.391 6.309) (width 0.2) (layer "F.Cu") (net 16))
 (segment (start 6.391 6.309) (end 4.682 6.309) (width 0.2) (layer "F.Cu") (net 16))
 (segment (start 20.421 3.709) (end 20.447 3.683) (width 0.2) (layer "F.Cu") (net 16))
 (via (at 20.447 3.683) (size 0.8) (drill 0.4) (layers "F.Cu" "B.Cu") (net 16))
 (segment (start 20.447 3.683) (end 20.447 10.287) (width 0.2) (layer "B.Cu") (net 16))
 (segment (start 20.447 10.287) (end 22.86 12.7) (width 0.2) (layer "B.Cu") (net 16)))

